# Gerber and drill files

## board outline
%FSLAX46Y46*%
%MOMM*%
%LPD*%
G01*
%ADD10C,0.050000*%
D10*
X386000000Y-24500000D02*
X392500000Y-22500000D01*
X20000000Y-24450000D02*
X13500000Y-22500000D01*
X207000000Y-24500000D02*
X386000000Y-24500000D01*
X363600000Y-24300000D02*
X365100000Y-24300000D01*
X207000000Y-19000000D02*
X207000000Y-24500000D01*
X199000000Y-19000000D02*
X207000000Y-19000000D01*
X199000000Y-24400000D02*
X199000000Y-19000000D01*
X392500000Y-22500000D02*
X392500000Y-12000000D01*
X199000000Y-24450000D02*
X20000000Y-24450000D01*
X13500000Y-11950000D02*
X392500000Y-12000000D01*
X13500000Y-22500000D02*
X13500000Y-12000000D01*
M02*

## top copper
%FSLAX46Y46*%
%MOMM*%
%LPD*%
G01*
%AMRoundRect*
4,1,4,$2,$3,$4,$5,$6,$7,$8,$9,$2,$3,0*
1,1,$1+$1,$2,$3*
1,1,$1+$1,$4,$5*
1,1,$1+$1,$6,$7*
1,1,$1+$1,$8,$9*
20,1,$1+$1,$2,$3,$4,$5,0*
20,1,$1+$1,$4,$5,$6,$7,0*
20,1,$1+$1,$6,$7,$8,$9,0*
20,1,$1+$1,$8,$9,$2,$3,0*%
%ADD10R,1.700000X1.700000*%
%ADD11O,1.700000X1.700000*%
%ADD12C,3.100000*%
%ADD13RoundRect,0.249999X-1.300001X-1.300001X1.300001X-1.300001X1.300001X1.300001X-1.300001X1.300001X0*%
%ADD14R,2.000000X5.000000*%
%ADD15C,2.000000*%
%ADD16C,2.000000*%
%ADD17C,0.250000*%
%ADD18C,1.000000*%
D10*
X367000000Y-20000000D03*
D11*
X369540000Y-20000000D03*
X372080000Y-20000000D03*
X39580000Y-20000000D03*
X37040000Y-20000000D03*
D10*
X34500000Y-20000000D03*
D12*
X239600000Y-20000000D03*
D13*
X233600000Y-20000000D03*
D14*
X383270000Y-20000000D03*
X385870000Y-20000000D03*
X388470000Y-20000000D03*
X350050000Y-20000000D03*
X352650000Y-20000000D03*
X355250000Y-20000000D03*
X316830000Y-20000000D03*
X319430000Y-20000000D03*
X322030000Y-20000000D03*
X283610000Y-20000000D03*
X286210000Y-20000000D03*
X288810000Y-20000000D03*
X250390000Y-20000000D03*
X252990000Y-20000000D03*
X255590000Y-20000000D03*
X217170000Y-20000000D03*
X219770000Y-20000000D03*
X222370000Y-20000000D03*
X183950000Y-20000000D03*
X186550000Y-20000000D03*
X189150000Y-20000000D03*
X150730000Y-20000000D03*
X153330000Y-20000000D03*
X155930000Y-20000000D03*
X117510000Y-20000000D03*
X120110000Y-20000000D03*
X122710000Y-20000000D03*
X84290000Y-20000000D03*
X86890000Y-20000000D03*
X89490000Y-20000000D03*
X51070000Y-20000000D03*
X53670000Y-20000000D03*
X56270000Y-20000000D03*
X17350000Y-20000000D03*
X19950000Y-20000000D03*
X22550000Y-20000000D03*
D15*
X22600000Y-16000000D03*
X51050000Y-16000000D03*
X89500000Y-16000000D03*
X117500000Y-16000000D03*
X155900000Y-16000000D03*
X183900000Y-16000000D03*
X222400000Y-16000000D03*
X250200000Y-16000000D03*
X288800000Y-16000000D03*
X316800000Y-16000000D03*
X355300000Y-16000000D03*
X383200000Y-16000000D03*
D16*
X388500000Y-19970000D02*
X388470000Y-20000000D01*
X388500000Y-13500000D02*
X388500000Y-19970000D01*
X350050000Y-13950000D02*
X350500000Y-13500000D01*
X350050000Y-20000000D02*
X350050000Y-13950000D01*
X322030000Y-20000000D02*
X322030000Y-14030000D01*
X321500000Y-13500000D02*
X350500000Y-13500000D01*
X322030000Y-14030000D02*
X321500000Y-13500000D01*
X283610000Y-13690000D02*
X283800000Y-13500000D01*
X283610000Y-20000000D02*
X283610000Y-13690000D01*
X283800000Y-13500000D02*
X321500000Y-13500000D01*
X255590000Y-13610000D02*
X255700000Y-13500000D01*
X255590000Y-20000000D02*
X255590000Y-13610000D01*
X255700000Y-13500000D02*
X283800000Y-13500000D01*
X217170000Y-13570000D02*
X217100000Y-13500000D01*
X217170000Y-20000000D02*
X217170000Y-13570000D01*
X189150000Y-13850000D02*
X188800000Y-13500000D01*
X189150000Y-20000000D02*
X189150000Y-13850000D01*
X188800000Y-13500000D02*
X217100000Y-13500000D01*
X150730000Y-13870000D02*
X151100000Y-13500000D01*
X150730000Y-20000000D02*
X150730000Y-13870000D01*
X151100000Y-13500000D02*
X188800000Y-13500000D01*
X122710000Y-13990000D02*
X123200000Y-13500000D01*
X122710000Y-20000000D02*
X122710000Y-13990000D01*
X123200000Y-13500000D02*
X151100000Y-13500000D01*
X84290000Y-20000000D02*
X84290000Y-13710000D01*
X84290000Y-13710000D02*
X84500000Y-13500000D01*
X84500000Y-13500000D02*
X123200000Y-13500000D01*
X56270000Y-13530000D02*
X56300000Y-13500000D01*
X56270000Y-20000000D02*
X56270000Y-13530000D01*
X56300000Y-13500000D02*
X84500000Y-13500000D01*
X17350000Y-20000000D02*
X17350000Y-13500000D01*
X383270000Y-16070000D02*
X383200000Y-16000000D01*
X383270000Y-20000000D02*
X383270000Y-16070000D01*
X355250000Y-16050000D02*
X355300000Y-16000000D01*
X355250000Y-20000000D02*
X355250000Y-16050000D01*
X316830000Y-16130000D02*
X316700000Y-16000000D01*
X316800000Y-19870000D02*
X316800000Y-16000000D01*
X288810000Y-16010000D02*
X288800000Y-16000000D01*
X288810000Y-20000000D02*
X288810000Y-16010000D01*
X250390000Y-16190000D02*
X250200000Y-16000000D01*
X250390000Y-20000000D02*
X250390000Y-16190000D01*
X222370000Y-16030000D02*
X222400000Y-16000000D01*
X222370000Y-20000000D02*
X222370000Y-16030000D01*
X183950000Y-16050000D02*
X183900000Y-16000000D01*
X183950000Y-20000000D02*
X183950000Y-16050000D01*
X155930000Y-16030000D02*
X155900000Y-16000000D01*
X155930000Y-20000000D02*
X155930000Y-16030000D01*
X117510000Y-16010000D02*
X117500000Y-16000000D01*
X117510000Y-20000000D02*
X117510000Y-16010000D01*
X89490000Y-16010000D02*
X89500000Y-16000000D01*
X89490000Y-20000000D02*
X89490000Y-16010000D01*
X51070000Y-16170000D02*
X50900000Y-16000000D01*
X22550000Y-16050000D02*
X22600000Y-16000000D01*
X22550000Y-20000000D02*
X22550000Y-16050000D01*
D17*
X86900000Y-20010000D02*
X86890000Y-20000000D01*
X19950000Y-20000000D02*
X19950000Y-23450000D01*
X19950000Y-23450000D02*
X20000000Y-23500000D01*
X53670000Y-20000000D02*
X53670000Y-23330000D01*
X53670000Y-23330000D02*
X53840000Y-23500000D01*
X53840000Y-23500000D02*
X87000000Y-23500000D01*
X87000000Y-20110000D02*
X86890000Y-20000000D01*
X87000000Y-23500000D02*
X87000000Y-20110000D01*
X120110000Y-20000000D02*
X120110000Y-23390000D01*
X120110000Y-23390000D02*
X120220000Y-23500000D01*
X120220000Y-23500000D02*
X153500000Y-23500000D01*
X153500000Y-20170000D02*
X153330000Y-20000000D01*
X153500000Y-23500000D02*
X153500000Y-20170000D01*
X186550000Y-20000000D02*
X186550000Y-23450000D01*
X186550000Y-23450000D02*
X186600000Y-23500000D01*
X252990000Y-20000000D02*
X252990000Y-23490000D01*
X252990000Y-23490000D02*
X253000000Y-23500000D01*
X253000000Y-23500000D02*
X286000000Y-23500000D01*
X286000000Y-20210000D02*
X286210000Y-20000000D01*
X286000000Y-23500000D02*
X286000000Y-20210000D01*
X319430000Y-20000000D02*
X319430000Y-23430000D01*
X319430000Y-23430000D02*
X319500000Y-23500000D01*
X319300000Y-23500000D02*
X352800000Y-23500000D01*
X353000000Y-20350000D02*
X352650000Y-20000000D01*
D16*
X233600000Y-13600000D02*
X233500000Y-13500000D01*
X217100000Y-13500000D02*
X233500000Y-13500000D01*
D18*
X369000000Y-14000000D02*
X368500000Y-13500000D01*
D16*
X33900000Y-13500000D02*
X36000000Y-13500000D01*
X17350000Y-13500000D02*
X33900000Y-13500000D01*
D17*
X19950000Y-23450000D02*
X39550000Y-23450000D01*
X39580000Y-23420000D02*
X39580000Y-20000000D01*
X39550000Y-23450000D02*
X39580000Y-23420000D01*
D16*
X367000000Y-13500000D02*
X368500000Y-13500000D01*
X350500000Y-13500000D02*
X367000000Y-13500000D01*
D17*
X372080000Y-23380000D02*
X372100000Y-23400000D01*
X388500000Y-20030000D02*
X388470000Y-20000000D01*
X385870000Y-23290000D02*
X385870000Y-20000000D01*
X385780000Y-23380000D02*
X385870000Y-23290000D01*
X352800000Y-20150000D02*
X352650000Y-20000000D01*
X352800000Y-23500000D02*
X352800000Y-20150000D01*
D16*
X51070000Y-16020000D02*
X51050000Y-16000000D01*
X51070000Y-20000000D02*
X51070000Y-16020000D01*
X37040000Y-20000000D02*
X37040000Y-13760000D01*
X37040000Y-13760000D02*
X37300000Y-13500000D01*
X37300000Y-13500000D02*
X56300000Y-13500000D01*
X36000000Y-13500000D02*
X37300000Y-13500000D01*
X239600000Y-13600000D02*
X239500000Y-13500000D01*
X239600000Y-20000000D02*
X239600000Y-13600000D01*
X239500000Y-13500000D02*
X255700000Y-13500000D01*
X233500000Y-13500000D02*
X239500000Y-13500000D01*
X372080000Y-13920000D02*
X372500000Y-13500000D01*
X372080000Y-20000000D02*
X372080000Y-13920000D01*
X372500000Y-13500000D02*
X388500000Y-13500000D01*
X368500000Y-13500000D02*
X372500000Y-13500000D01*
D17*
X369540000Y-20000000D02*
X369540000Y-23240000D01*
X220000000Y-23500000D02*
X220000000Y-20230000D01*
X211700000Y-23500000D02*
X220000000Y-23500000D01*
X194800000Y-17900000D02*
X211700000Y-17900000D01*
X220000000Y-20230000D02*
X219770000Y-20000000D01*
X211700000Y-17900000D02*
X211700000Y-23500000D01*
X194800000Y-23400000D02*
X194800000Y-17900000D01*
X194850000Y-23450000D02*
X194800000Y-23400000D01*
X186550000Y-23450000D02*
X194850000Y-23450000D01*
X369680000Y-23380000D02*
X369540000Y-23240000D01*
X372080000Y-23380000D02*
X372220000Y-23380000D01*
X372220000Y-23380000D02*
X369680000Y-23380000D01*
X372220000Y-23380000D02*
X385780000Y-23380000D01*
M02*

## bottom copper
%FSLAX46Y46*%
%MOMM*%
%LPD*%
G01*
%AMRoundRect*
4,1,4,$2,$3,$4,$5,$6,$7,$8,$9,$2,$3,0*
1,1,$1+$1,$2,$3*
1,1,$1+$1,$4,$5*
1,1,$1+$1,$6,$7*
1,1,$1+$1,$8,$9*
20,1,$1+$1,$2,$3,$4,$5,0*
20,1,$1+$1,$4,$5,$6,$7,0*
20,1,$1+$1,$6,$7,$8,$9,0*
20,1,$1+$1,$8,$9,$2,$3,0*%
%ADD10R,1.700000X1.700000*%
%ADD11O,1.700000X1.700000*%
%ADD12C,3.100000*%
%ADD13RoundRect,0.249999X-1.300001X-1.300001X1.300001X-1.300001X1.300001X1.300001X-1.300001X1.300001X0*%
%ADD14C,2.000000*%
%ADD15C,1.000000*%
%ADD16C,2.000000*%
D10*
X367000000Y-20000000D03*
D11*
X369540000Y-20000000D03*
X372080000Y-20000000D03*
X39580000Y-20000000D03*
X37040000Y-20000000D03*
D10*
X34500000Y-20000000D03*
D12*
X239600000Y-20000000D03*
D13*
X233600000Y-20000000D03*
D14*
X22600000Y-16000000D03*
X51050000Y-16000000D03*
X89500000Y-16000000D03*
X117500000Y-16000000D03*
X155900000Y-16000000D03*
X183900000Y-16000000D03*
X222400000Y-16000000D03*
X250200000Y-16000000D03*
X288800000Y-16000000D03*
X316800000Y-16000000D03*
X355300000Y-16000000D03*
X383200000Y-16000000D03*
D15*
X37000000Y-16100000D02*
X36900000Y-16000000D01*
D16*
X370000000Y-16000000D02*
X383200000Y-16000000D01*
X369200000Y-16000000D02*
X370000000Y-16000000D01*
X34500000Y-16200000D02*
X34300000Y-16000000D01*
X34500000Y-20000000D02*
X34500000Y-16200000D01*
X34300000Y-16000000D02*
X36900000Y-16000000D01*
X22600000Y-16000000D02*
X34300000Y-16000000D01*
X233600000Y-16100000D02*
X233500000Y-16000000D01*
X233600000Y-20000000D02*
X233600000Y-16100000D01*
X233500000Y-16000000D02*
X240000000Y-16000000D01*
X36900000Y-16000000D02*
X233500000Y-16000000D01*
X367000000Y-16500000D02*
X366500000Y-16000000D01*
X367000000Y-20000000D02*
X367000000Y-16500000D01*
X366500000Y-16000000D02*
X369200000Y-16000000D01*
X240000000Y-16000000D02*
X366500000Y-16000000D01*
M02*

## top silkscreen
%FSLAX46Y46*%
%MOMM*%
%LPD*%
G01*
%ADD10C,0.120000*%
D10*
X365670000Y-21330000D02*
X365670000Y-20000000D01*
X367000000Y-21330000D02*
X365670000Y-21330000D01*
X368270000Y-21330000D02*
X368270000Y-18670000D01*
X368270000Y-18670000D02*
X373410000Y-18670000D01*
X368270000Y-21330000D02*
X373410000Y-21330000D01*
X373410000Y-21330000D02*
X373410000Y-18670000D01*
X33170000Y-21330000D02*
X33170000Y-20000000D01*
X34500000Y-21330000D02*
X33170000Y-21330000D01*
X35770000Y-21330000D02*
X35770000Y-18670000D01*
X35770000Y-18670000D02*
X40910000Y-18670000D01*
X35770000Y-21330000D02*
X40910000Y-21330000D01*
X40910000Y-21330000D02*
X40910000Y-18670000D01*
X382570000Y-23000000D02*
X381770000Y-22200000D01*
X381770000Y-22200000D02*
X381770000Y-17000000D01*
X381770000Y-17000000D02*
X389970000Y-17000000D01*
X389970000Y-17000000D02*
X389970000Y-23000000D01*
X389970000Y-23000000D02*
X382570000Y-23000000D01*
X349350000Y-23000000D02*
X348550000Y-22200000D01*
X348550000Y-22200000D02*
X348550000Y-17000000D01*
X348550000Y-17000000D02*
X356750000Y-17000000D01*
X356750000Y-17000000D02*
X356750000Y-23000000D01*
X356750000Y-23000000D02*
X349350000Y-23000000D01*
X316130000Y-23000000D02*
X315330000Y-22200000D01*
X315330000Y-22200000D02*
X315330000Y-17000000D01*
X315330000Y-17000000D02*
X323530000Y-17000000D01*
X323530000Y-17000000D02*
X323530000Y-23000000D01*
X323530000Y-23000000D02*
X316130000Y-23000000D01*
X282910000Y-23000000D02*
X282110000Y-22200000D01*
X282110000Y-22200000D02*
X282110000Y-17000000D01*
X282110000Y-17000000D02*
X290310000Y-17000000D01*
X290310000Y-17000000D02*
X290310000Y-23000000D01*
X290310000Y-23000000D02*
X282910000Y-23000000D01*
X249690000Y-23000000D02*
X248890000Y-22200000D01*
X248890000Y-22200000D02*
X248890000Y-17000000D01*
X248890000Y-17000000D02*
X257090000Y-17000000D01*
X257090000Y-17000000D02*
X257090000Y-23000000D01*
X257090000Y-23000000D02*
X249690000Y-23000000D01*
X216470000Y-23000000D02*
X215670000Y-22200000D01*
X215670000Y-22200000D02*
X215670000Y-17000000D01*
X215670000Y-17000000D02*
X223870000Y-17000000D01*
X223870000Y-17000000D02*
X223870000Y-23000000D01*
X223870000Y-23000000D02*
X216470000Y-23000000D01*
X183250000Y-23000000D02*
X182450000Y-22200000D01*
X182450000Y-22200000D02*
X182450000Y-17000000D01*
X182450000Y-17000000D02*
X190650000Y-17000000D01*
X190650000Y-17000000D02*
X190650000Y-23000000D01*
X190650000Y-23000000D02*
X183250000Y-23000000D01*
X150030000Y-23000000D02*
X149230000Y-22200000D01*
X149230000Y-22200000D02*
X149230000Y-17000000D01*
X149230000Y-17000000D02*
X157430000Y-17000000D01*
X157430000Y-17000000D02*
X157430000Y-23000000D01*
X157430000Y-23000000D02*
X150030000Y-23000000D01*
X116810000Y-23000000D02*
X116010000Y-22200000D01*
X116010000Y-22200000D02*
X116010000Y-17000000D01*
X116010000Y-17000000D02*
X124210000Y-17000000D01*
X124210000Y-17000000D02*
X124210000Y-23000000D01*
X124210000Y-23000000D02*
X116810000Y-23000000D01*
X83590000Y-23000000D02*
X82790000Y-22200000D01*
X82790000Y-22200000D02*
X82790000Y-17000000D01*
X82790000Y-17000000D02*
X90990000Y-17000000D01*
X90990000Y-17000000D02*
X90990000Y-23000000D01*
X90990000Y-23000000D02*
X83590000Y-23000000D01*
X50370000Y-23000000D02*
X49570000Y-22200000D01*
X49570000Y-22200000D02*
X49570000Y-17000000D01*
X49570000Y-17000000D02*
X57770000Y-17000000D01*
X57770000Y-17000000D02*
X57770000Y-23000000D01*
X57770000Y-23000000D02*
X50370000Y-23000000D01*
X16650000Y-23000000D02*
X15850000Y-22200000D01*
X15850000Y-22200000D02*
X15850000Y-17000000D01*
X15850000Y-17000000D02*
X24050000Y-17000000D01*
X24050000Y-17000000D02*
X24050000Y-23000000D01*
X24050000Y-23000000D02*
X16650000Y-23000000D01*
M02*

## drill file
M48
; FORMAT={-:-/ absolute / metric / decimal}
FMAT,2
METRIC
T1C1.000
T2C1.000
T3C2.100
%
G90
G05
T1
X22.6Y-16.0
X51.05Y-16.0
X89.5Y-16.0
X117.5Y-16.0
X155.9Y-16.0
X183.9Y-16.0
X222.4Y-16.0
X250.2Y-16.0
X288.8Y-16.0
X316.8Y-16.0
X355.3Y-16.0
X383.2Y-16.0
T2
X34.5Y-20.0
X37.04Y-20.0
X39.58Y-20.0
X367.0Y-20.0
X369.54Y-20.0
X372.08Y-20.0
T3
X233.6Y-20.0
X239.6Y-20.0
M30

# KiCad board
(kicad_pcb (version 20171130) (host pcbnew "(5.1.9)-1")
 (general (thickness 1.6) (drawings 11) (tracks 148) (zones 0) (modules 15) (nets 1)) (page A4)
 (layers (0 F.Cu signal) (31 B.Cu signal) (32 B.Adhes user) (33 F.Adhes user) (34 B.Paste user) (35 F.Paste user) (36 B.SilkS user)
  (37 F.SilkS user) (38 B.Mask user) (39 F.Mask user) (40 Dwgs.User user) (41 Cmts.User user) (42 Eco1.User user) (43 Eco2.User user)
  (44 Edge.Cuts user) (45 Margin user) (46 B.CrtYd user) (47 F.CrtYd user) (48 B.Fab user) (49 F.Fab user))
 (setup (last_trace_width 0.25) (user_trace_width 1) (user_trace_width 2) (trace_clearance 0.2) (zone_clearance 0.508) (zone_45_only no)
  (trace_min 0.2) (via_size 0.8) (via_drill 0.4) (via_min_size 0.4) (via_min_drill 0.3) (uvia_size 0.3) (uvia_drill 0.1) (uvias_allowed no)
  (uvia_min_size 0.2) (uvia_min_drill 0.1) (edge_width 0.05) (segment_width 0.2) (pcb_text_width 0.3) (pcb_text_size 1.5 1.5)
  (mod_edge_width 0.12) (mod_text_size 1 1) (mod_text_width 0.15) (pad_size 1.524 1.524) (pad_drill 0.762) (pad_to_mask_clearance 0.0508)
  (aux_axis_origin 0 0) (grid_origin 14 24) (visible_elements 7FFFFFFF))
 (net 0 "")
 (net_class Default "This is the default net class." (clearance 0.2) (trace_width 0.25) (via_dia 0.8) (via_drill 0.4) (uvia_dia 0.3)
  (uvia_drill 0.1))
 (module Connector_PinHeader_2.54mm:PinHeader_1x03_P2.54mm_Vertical (layer F.Cu) (at 367 20 90)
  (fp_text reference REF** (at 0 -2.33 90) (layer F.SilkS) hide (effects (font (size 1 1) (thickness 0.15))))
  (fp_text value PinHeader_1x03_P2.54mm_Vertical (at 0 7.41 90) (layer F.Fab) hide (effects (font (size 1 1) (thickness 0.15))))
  (fp_line (start -1.33 -1.33) (end 0 -1.33) (layer F.SilkS) (width 0.12))
  (fp_line (start -1.33 0) (end -1.33 -1.33) (layer F.SilkS) (width 0.12))
  (fp_line (start -1.33 1.27) (end 1.33 1.27) (layer F.SilkS) (width 0.12))
  (fp_line (start 1.33 1.27) (end 1.33 6.41) (layer F.SilkS) (width 0.12))
  (fp_line (start -1.33 1.27) (end -1.33 6.41) (layer F.SilkS) (width 0.12))
  (fp_line (start -1.33 6.41) (end 1.33 6.41) (layer F.SilkS) (width 0.12))
  (pad 1 thru_hole rect (at 0 0 90) (size 1.7 1.7) (drill 1) (layers *.Cu *.Mask))
  (pad 2 thru_hole oval (at 0 2.54 90) (size 1.7 1.7) (drill 1) (layers *.Cu *.Mask))
  (pad 3 thru_hole oval (at 0 5.08 90) (size 1.7 1.7) (drill 1) (layers *.Cu *.Mask)))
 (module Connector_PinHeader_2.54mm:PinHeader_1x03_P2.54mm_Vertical (layer F.Cu) (at 34.5 20 90)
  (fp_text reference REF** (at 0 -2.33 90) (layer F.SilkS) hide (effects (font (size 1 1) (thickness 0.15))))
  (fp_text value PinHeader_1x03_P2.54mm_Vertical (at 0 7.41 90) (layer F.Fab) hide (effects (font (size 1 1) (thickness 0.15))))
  (fp_line (start -1.33 -1.33) (end 0 -1.33) (layer F.SilkS) (width 0.12))
  (fp_line (start -1.33 0) (end -1.33 -1.33) (layer F.SilkS) (width 0.12))
  (fp_line (start -1.33 1.27) (end 1.33 1.27) (layer F.SilkS) (width 0.12))
  (fp_line (start 1.33 1.27) (end 1.33 6.41) (layer F.SilkS) (width 0.12))
  (fp_line (start -1.33 1.27) (end -1.33 6.41) (layer F.SilkS) (width 0.12))
  (fp_line (start -1.33 6.41) (end 1.33 6.41) (layer F.SilkS) (width 0.12))
  (pad 3 thru_hole oval (at 0 5.08 90) (size 1.7 1.7) (drill 1) (layers *.Cu *.Mask))
  (pad 2 thru_hole oval (at 0 2.54 90) (size 1.7 1.7) (drill 1) (layers *.Cu *.Mask))
  (pad 1 thru_hole rect (at 0 0 90) (size 1.7 1.7) (drill 1) (layers *.Cu *.Mask)))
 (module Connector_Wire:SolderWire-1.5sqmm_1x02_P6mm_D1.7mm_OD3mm (layer F.Cu) (at 233.6 20)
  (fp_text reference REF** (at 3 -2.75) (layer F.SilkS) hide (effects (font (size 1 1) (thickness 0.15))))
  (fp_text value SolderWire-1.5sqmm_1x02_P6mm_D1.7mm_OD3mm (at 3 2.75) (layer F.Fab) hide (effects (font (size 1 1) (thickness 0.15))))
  (pad 2 thru_hole circle (at 6 0) (size 3.1 3.1) (drill 2.1) (layers *.Cu *.Mask))
  (pad 1 thru_hole roundrect (at 0 0) (size 3.1 3.1) (drill 2.1) (layers *.Cu *.Mask) (roundrect_rratio 0.08064499999999999)))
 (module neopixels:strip (layer F.Cu) (at 385.87 20)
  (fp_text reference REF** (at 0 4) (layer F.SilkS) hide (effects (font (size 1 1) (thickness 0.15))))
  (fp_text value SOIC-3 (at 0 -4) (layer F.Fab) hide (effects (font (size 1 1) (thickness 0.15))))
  (fp_line (start -3.3 3) (end -4.1 2.2) (layer F.SilkS) (width 0.12))
  (fp_line (start -4.1 2.2) (end -4.1 -3) (layer F.SilkS) (width 0.12))
  (fp_line (start -4.1 -3) (end 4.1 -3) (layer F.SilkS) (width 0.12))
  (fp_line (start 4.1 -3) (end 4.1 3) (layer F.SilkS) (width 0.12))
  (fp_line (start 4.1 3) (end -3.3 3) (layer F.SilkS) (width 0.12))
  (pad 1 smd rect (at -2.6 0) (size 2 5) (layers F.Cu F.Paste F.Mask))
  (pad 2 smd rect (at 0 0) (size 2 5) (layers F.Cu F.Paste F.Mask))
  (pad 3 smd rect (at 2.6 0) (size 2 5) (layers F.Cu F.Paste F.Mask)))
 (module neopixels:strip (layer F.Cu) (at 352.65 20)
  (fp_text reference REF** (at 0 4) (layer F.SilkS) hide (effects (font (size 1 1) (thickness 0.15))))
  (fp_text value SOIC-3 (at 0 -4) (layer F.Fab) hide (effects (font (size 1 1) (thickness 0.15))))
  (fp_line (start -3.3 3) (end -4.1 2.2) (layer F.SilkS) (width 0.12))
  (fp_line (start -4.1 2.2) (end -4.1 -3) (layer F.SilkS) (width 0.12))
  (fp_line (start -4.1 -3) (end 4.1 -3) (layer F.SilkS) (width 0.12))
  (fp_line (start 4.1 -3) (end 4.1 3) (layer F.SilkS) (width 0.12))
  (fp_line (start 4.1 3) (end -3.3 3) (layer F.SilkS) (width 0.12))
  (pad 1 smd rect (at -2.6 0) (size 2 5) (layers F.Cu F.Paste F.Mask))
  (pad 2 smd rect (at 0 0) (size 2 5) (layers F.Cu F.Paste F.Mask))
  (pad 3 smd rect (at 2.6 0) (size 2 5) (layers F.Cu F.Paste F.Mask)))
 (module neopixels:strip (layer F.Cu) (at 319.43 20)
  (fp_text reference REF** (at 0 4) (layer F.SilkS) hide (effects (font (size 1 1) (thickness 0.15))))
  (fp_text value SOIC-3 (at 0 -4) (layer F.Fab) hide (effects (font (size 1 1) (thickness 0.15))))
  (fp_line (start -3.3 3) (end -4.1 2.2) (layer F.SilkS) (width 0.12))
  (fp_line (start -4.1 2.2) (end -4.1 -3) (layer F.SilkS) (width 0.12))
  (fp_line (start -4.1 -3) (end 4.1 -3) (layer F.SilkS) (width 0.12))
  (fp_line (start 4.1 -3) (end 4.1 3) (layer F.SilkS) (width 0.12))
  (fp_line (start 4.1 3) (end -3.3 3) (layer F.SilkS) (width 0.12))
  (pad 1 smd rect (at -2.6 0) (size 2 5) (layers F.Cu F.Paste F.Mask))
  (pad 2 smd rect (at 0 0) (size 2 5) (layers F.Cu F.Paste F.Mask))
  (pad 3 smd rect (at 2.6 0) (size 2 5) (layers F.Cu F.Paste F.Mask)))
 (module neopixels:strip (layer F.Cu) (at 286.21 20)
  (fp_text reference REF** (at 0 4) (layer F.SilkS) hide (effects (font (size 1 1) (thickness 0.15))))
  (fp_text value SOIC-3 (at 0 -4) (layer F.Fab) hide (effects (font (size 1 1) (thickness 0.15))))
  (fp_line (start -3.3 3) (end -4.1 2.2) (layer F.SilkS) (width 0.12))
  (fp_line (start -4.1 2.2) (end -4.1 -3) (layer F.SilkS) (width 0.12))
  (fp_line (start -4.1 -3) (end 4.1 -3) (layer F.SilkS) (width 0.12))
  (fp_line (start 4.1 -3) (end 4.1 3) (layer F.SilkS) (width 0.12))
  (fp_line (start 4.1 3) (end -3.3 3) (layer F.SilkS) (width 0.12))
  (pad 1 smd rect (at -2.6 0) (size 2 5) (layers F.Cu F.Paste F.Mask))
  (pad 2 smd rect (at 0 0) (size 2 5) (layers F.Cu F.Paste F.Mask))
  (pad 3 smd rect (at 2.6 0) (size 2 5) (layers F.Cu F.Paste F.Mask)))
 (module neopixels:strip (layer F.Cu) (at 252.99 20)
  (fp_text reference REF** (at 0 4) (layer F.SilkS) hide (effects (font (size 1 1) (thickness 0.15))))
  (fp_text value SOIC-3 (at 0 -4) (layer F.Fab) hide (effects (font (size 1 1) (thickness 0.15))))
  (fp_line (start -3.3 3) (end -4.1 2.2) (layer F.SilkS) (width 0.12))
  (fp_line (start -4.1 2.2) (end -4.1 -3) (layer F.SilkS) (width 0.12))
  (fp_line (start -4.1 -3) (end 4.1 -3) (layer F.SilkS) (width 0.12))
  (fp_line (start 4.1 -3) (end 4.1 3) (layer F.SilkS) (width 0.12))
  (fp_line (start 4.1 3) (end -3.3 3) (layer F.SilkS) (width 0.12))
  (pad 1 smd rect (at -2.6 0) (size 2 5) (layers F.Cu F.Paste F.Mask))
  (pad 2 smd rect (at 0 0) (size 2 5) (layers F.Cu F.Paste F.Mask))
  (pad 3 smd rect (at 2.6 0) (size 2 5) (layers F.Cu F.Paste F.Mask)))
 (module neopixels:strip (layer F.Cu) (at 219.77 20)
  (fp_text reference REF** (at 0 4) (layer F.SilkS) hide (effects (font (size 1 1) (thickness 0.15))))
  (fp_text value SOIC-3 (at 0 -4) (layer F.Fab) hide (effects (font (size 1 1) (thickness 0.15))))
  (fp_line (start -3.3 3) (end -4.1 2.2) (layer F.SilkS) (width 0.12))
  (fp_line (start -4.1 2.2) (end -4.1 -3) (layer F.SilkS) (width 0.12))
  (fp_line (start -4.1 -3) (end 4.1 -3) (layer F.SilkS) (width 0.12))
  (fp_line (start 4.1 -3) (end 4.1 3) (layer F.SilkS) (width 0.12))
  (fp_line (start 4.1 3) (end -3.3 3) (layer F.SilkS) (width 0.12))
  (pad 1 smd rect (at -2.6 0) (size 2 5) (layers F.Cu F.Paste F.Mask))
  (pad 2 smd rect (at 0 0) (size 2 5) (layers F.Cu F.Paste F.Mask))
  (pad 3 smd rect (at 2.6 0) (size 2 5) (layers F.Cu F.Paste F.Mask)))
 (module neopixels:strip (layer F.Cu) (at 186.55 20)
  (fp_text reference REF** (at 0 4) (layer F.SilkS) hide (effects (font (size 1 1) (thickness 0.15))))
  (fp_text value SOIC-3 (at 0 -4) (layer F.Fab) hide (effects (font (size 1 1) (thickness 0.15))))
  (fp_line (start -3.3 3) (end -4.1 2.2) (layer F.SilkS) (width 0.12))
  (fp_line (start -4.1 2.2) (end -4.1 -3) (layer F.SilkS) (width 0.12))
  (fp_line (start -4.1 -3) (end 4.1 -3) (layer F.SilkS) (width 0.12))
  (fp_line (start 4.1 -3) (end 4.1 3) (layer F.SilkS) (width 0.12))
  (fp_line (start 4.1 3) (end -3.3 3) (layer F.SilkS) (width 0.12))
  (pad 1 smd rect (at -2.6 0) (size 2 5) (layers F.Cu F.Paste F.Mask))
  (pad 2 smd rect (at 0 0) (size 2 5) (layers F.Cu F.Paste F.Mask))
  (pad 3 smd rect (at 2.6 0) (size 2 5) (layers F.Cu F.Paste F.Mask)))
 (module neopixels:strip (layer F.Cu) (at 153.33 20)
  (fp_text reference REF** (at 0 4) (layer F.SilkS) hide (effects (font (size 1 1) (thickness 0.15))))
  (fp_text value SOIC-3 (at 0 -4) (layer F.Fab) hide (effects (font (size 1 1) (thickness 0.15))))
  (fp_line (start -3.3 3) (end -4.1 2.2) (layer F.SilkS) (width 0.12))
  (fp_line (start -4.1 2.2) (end -4.1 -3) (layer F.SilkS) (width 0.12))
  (fp_line (start -4.1 -3) (end 4.1 -3) (layer F.SilkS) (width 0.12))
  (fp_line (start 4.1 -3) (end 4.1 3) (layer F.SilkS) (width 0.12))
  (fp_line (start 4.1 3) (end -3.3 3) (layer F.SilkS) (width 0.12))
  (pad 1 smd rect (at -2.6 0) (size 2 5) (layers F.Cu F.Paste F.Mask))
  (pad 2 smd rect (at 0 0) (size 2 5) (layers F.Cu F.Paste F.Mask))
  (pad 3 smd rect (at 2.6 0) (size 2 5) (layers F.Cu F.Paste F.Mask)))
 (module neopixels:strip (layer F.Cu) (at 120.11 20)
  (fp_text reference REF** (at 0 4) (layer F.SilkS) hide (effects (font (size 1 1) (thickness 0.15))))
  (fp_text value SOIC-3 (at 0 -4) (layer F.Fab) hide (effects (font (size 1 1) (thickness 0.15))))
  (fp_line (start -3.3 3) (end -4.1 2.2) (layer F.SilkS) (width 0.12))
  (fp_line (start -4.1 2.2) (end -4.1 -3) (layer F.SilkS) (width 0.12))
  (fp_line (start -4.1 -3) (end 4.1 -3) (layer F.SilkS) (width 0.12))
  (fp_line (start 4.1 -3) (end 4.1 3) (layer F.SilkS) (width 0.12))
  (fp_line (start 4.1 3) (end -3.3 3) (layer F.SilkS) (width 0.12))
  (pad 1 smd rect (at -2.6 0) (size 2 5) (layers F.Cu F.Paste F.Mask))
  (pad 2 smd rect (at 0 0) (size 2 5) (layers F.Cu F.Paste F.Mask))
  (pad 3 smd rect (at 2.6 0) (size 2 5) (layers F.Cu F.Paste F.Mask)))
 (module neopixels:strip (layer F.Cu) (at 86.89 20)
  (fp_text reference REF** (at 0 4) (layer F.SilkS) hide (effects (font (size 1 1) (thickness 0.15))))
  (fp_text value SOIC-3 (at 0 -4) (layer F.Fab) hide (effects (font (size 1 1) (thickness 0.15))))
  (fp_line (start -3.3 3) (end -4.1 2.2) (layer F.SilkS) (width 0.12))
  (fp_line (start -4.1 2.2) (end -4.1 -3) (layer F.SilkS) (width 0.12))
  (fp_line (start -4.1 -3) (end 4.1 -3) (layer F.SilkS) (width 0.12))
  (fp_line (start 4.1 -3) (end 4.1 3) (layer F.SilkS) (width 0.12))
  (fp_line (start 4.1 3) (end -3.3 3) (layer F.SilkS) (width 0.12))
  (pad 1 smd rect (at -2.6 0) (size 2 5) (layers F.Cu F.Paste F.Mask))
  (pad 2 smd rect (at 0 0) (size 2 5) (layers F.Cu F.Paste F.Mask))
  (pad 3 smd rect (at 2.6 0) (size 2 5) (layers F.Cu F.Paste F.Mask)))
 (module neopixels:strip (layer F.Cu) (at 53.67 20)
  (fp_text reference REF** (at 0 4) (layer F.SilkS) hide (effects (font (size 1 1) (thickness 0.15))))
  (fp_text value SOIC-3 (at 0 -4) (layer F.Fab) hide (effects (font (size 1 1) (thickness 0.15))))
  (fp_line (start -3.3 3) (end -4.1 2.2) (layer F.SilkS) (width 0.12))
  (fp_line (start -4.1 2.2) (end -4.1 -3) (layer F.SilkS) (width 0.12))
  (fp_line (start -4.1 -3) (end 4.1 -3) (layer F.SilkS) (width 0.12))
  (fp_line (start 4.1 -3) (end 4.1 3) (layer F.SilkS) (width 0.12))
  (fp_line (start 4.1 3) (end -3.3 3) (layer F.SilkS) (width 0.12))
  (pad 1 smd rect (at -2.6 0) (size 2 5) (layers F.Cu F.Paste F.Mask))
  (pad 2 smd rect (at 0 0) (size 2 5) (layers F.Cu F.Paste F.Mask))
  (pad 3 smd rect (at 2.6 0) (size 2 5) (layers F.Cu F.Paste F.Mask)))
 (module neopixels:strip (layer F.Cu) (at 19.95 20)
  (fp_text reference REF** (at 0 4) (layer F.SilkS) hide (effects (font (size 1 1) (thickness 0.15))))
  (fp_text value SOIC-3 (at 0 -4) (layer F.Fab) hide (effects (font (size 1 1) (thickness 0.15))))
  (fp_line (start -3.3 3) (end -4.1 2.2) (layer F.SilkS) (width 0.12))
  (fp_line (start -4.1 2.2) (end -4.1 -3) (layer F.SilkS) (width 0.12))
  (fp_line (start -4.1 -3) (end 4.1 -3) (layer F.SilkS) (width 0.12))
  (fp_line (start 4.1 -3) (end 4.1 3) (layer F.SilkS) (width 0.12))
  (fp_line (start 4.1 3) (end -3.3 3) (layer F.SilkS) (width 0.12))
  (pad 1 smd rect (at -2.6 0) (size 2 5) (layers F.Cu F.Paste F.Mask))
  (pad 2 smd rect (at 0 0) (size 2 5) (layers F.Cu F.Paste F.Mask))
  (pad 3 smd rect (at 2.6 0) (size 2 5) (layers F.Cu F.Paste F.Mask)))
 (gr_line (start 386 24.5) (end 392.5 22.5) (layer Edge.Cuts) (width 0.05))
 (gr_line (start 20 24.45) (end 13.5 22.5) (layer Edge.Cuts) (width 0.05))
 (gr_line (start 207 24.5) (end 386 24.5) (layer Edge.Cuts) (width 0.05))
 (gr_line (start 363.6 24.3) (end 365.1 24.3) (layer Edge.Cuts) (width 0.05))
 (gr_line (start 207 19) (end 207 24.5) (layer Edge.Cuts) (width 0.05))
 (gr_line (start 199 19) (end 207 19) (layer Edge.Cuts) (width 0.05))
 (gr_line (start 199 24.4) (end 199 19) (layer Edge.Cuts) (width 0.05))
 (gr_line (start 392.5 22.5) (end 392.5 12) (layer Edge.Cuts) (width 0.05))
 (gr_line (start 199 24.45) (end 20 24.45) (layer Edge.Cuts) (width 0.05))
 (gr_line (start 13.5 11.95) (end 392.5 12) (layer Edge.Cuts) (width 0.05))
 (gr_line (start 13.5 22.5) (end 13.5 12) (layer Edge.Cuts) (width 0.05))
 (segment (start 388.5 19.97) (end 388.47 20) (width 2) (layer F.Cu) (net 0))
 (segment (start 388.5 13.5) (end 388.5 19.97) (width 2) (layer F.Cu) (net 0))
 (segment (start 350.05 13.95) (end 350.5 13.5) (width 2) (layer F.Cu) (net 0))
 (segment (start 350.05 20) (end 350.05 13.95) (width 2) (layer F.Cu) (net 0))
 (segment (start 322.03 20) (end 322.03 14.03) (width 2) (layer F.Cu) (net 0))
 (segment (start 321.5 13.5) (end 350.5 13.5) (width 2) (layer F.Cu) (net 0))
 (segment (start 322.03 14.03) (end 321.5 13.5) (width 2) (layer F.Cu) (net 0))
 (segment (start 283.61 13.69) (end 283.8 13.5) (width 2) (layer F.Cu) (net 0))
 (segment (start 283.61 20) (end 283.61 13.69) (width 2) (layer F.Cu) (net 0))
 (segment (start 283.8 13.5) (end 321.5 13.5) (width 2) (layer F.Cu) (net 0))
 (segment (start 255.59 13.61) (end 255.7 13.5) (width 2) (layer F.Cu) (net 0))
 (segment (start 255.59 20) (end 255.59 13.61) (width 2) (layer F.Cu) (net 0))
 (segment (start 255.7 13.5) (end 283.8 13.5) (width 2) (layer F.Cu) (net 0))
 (segment (start 217.17 13.57) (end 217.1 13.5) (width 2) (layer F.Cu) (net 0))
 (segment (start 217.17 20) (end 217.17 13.57) (width 2) (layer F.Cu) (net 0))
 (segment (start 189.15 13.85) (end 188.8 13.5) (width 2) (layer F.Cu) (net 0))
 (segment (start 189.15 20) (end 189.15 13.85) (width 2) (layer F.Cu) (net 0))
 (segment (start 188.8 13.5) (end 217.1 13.5) (width 2) (layer F.Cu) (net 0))
 (segment (start 150.73 13.87) (end 151.1 13.5) (width 2) (layer F.Cu) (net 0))
 (segment (start 150.73 20) (end 150.73 13.87) (width 2) (layer F.Cu) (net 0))
 (segment (start 151.1 13.5) (end 188.8 13.5) (width 2) (layer F.Cu) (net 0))
 (segment (start 122.71 13.99) (end 123.2 13.5) (width 2) (layer F.Cu) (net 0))
 (segment (start 122.71 20) (end 122.71 13.99) (width 2) (layer F.Cu) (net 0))
 (segment (start 123.2 13.5) (end 151.1 13.5) (width 2) (layer F.Cu) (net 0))
 (segment (start 84.29 20) (end 84.29 13.71) (width 2) (layer F.Cu) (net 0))
 (segment (start 84.29 13.71) (end 84.5 13.5) (width 2) (layer F.Cu) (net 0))
 (segment (start 84.5 13.5) (end 123.2 13.5) (width 2) (layer F.Cu) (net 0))
 (segment (start 56.27 13.53) (end 56.3 13.5) (width 2) (layer F.Cu) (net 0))
 (segment (start 56.27 20) (end 56.27 13.53) (width 2) (layer F.Cu) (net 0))
 (segment (start 56.3 13.5) (end 84.5 13.5) (width 2) (layer F.Cu) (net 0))
 (segment (start 17.35 20) (end 17.35 13.5) (width 2) (layer F.Cu) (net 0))
 (via (at 22.6 16) (size 2) (drill 1) (layers F.Cu B.Cu) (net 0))
 (via (at 51.05 16) (size 2) (drill 1) (layers F.Cu B.Cu) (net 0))
 (via (at 89.5 16) (size 2) (drill 1) (layers F.Cu B.Cu) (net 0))
 (via (at 117.5 16) (size 2) (drill 1) (layers F.Cu B.Cu) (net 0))
 (via (at 155.9 16) (size 2) (drill 1) (layers F.Cu B.Cu) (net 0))
 (via (at 183.9 16) (size 2) (drill 1) (layers F.Cu B.Cu) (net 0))
 (via (at 222.4 16) (size 2) (drill 1) (layers F.Cu B.Cu) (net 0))
 (via (at 250.2 16) (size 2) (drill 1) (layers F.Cu B.Cu) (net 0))
 (via (at 288.8 16) (size 2) (drill 1) (layers F.Cu B.Cu) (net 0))
 (via (at 316.8 16) (size 2) (drill 1) (layers F.Cu B.Cu) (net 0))
 (via (at 355.3 16) (size 2) (drill 1) (layers F.Cu B.Cu) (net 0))
 (via (at 383.2 16) (size 2) (drill 1) (layers F.Cu B.Cu) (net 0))
 (segment (start 383.27 16.07) (end 383.2 16) (width 2) (layer F.Cu) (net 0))
 (segment (start 383.27 20) (end 383.27 16.07) (width 2) (layer F.Cu) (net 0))
 (segment (start 355.25 16.05) (end 355.3 16) (width 2) (layer F.Cu) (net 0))
 (segment (start 355.25 20) (end 355.25 16.05) (width 2) (layer F.Cu) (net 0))
 (segment (start 316.83 16.13) (end 316.7 16) (width 2) (layer F.Cu) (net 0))
 (segment (start 316.8 19.87) (end 316.8 16) (width 2) (layer F.Cu) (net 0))
 (segment (start 288.81 16.01) (end 288.8 16) (width 2) (layer F.Cu) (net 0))
 (segment (start 288.81 20) (end 288.81 16.01) (width 2) (layer F.Cu) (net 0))
 (segment (start 250.39 16.19) (end 250.2 16) (width 2) (layer F.Cu) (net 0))
 (segment (start 250.39 20) (end 250.39 16.19) (width 2) (layer F.Cu) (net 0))
 (segment (start 222.37 16.03) (end 222.4 16) (width 2) (layer F.Cu) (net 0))
 (segment (start 222.37 20) (end 222.37 16.03) (width 2) (layer F.Cu) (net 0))
 (segment (start 183.95 16.05) (end 183.9 16) (width 2) (layer F.Cu) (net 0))
 (segment (start 183.95 20) (end 183.95 16.05) (width 2) (layer F.Cu) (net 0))
 (segment (start 155.93 16.03) (end 155.9 16) (width 2) (layer F.Cu) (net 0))
 (segment (start 155.93 20) (end 155.93 16.03) (width 2) (layer F.Cu) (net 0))
 (segment (start 117.51 16.01) (end 117.5 16) (width 2) (layer F.Cu) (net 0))
 (segment (start 117.51 20) (end 117.51 16.01) (width 2) (layer F.Cu) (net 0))
 (segment (start 89.49 16.01) (end 89.5 16) (width 2) (layer F.Cu) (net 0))
 (segment (start 89.49 20) (end 89.49 16.01) (width 2) (layer F.Cu) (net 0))
 (segment (start 51.07 16.17) (end 50.9 16) (width 2) (layer F.Cu) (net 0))
 (segment (start 22.55 16.05) (end 22.6 16) (width 2) (layer F.Cu) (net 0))
 (segment (start 22.55 20) (end 22.55 16.05) (width 2) (layer F.Cu) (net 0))
 (segment (start 37 16.1) (end 36.9 16) (width 1) (layer B.Cu) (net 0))
 (segment (start 86.9 20.01) (end 86.89 20) (width 0.25) (layer F.Cu) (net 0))
 (segment (start 19.95 20) (end 19.95 23.45) (width 0.25) (layer F.Cu) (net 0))
 (segment (start 19.95 23.45) (end 20 23.5) (width 0.25) (layer F.Cu) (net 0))
 (segment (start 53.67 20) (end 53.67 23.33) (width 0.25) (layer F.Cu) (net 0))
 (segment (start 53.67 23.33) (end 53.84 23.5) (width 0.25) (layer F.Cu) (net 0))
 (segment (start 53.84 23.5) (end 87 23.5) (width 0.25) (layer F.Cu) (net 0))
 (segment (start 87 20.11) (end 86.89 20) (width 0.25) (layer F.Cu) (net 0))
 (segment (start 87 23.5) (end 87 20.11) (width 0.25) (layer F.Cu) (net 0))
 (segment (start 120.11 20) (end 120.11 23.39) (width 0.25) (layer F.Cu) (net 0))
 (segment (start 120.11 23.39) (end 120.22 23.5) (width 0.25) (layer F.Cu) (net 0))
 (segment (start 120.22 23.5) (end 153.5 23.5) (width 0.25) (layer F.Cu) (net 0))
 (segment (start 153.5 20.17) (end 153.33 20) (width 0.25) (layer F.Cu) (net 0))
 (segment (start 153.5 23.5) (end 153.5 20.17) (width 0.25) (layer F.Cu) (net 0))
 (segment (start 186.55 20) (end 186.55 23.45) (width 0.25) (layer F.Cu) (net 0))
 (segment (start 186.55 23.45) (end 186.6 23.5) (width 0.25) (layer F.Cu) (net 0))
 (segment (start 252.99 20) (end 252.99 23.49) (width 0.25) (layer F.Cu) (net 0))
 (segment (start 252.99 23.49) (end 253 23.5) (width 0.25) (layer F.Cu) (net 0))
 (segment (start 253 23.5) (end 286 23.5) (width 0.25) (layer F.Cu) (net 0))
 (segment (start 286 20.21) (end 286.21 20) (width 0.25) (layer F.Cu) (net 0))
 (segment (start 286 23.5) (end 286 20.21) (width 0.25) (layer F.Cu) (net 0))
 (segment (start 319.43 20) (end 319.43 23.43) (width 0.25) (layer F.Cu) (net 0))
 (segment (start 319.43 23.43) (end 319.5 23.5) (width 0.25) (layer F.Cu) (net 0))
 (segment (start 319.3 23.5) (end 352.8 23.5) (width 0.25) (layer F.Cu) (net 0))
 (segment (start 353 20.35) (end 352.65 20) (width 0.25) (layer F.Cu) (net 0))
 (segment (start 233.6 13.6) (end 233.5 13.5) (width 2) (layer F.Cu) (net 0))
 (segment (start 217.1 13.5) (end 233.5 13.5) (width 2) (layer F.Cu) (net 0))
 (segment (start 369 14) (end 368.5 13.5) (width 1) (layer F.Cu) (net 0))
 (segment (start 370 16) (end 383.2 16) (width 2) (layer B.Cu) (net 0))
 (segment (start 33.9 13.5) (end 36 13.5) (width 2) (layer F.Cu) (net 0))
 (segment (start 17.35 13.5) (end 33.9 13.5) (width 2) (layer F.Cu) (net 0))
 (segment (start 19.95 23.45) (end 39.55 23.45) (width 0.25) (layer F.Cu) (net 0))
 (segment (start 39.58 23.42) (end 39.58 20) (width 0.25) (layer F.Cu) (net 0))
 (segment (start 39.55 23.45) (end 39.58 23.42) (width 0.25) (layer F.Cu) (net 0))
 (segment (start 367 13.5) (end 368.5 13.5) (width 2) (layer F.Cu) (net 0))
 (segment (start 350.5 13.5) (end 367 13.5) (width 2) (layer F.Cu) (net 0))
 (segment (start 369.2 16) (end 370 16) (width 2) (layer B.Cu) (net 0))
 (segment (start 372.08 23.38) (end 372.1 23.4) (width 0.25) (layer F.Cu) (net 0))
 (segment (start 388.5 20.03) (end 388.47 20) (width 0.25) (layer F.Cu) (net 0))
 (segment (start 385.87 23.29) (end 385.87 20) (width 0.25) (layer F.Cu) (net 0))
 (segment (start 385.78 23.38) (end 385.87 23.29) (width 0.25) (layer F.Cu) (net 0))
 (segment (start 352.8 20.15) (end 352.65 20) (width 0.25) (layer F.Cu) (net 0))
 (segment (start 352.8 23.5) (end 352.8 20.15) (width 0.25) (layer F.Cu) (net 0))
 (segment (start 51.07 16.02) (end 51.05 16) (width 2) (layer F.Cu) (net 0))
 (segment (start 51.07 20) (end 51.07 16.02) (width 2) (layer F.Cu) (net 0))
 (segment (start 34.5 16.2) (end 34.3 16) (width 2) (layer B.Cu) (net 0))
 (segment (start 34.5 20) (end 34.5 16.2) (width 2) (layer B.Cu) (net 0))
 (segment (start 34.3 16) (end 36.9 16) (width 2) (layer B.Cu) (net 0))
 (segment (start 22.6 16) (end 34.3 16) (width 2) (layer B.Cu) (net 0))
 (segment (start 37.04 20) (end 37.04 13.76) (width 2) (layer F.Cu) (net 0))
 (segment (start 37.04 13.76) (end 37.3 13.5) (width 2) (layer F.Cu) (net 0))
 (segment (start 37.3 13.5) (end 56.3 13.5) (width 2) (layer F.Cu) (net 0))
 (segment (start 36 13.5) (end 37.3 13.5) (width 2) (layer F.Cu) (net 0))
 (segment (start 233.6 16.1) (end 233.5 16) (width 2) (layer B.Cu) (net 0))
 (segment (start 233.6 20) (end 233.6 16.1) (width 2) (layer B.Cu) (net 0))
 (segment (start 233.5 16) (end 240 16) (width 2) (layer B.Cu) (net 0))
 (segment (start 36.9 16) (end 233.5 16) (width 2) (layer B.Cu) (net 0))
 (segment (start 239.6 13.6) (end 239.5 13.5) (width 2) (layer F.Cu) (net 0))
 (segment (start 239.6 20) (end 239.6 13.6) (width 2) (layer F.Cu) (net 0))
 (segment (start 239.5 13.5) (end 255.7 13.5) (width 2) (layer F.Cu) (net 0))
 (segment (start 233.5 13.5) (end 239.5 13.5) (width 2) (layer F.Cu) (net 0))
 (segment (start 367 16.5) (end 366.5 16) (width 2) (layer B.Cu) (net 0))
 (segment (start 367 20) (end 367 16.5) (width 2) (layer B.Cu) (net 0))
 (segment (start 366.5 16) (end 369.2 16) (width 2) (layer B.Cu) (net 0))
 (segment (start 240 16) (end 366.5 16) (width 2) (layer B.Cu) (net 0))
 (segment (start 372.08 13.92) (end 372.5 13.5) (width 2) (layer F.Cu) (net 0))
 (segment (start 372.08 20) (end 372.08 13.92) (width 2) (layer F.Cu) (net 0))
 (segment (start 372.5 13.5) (end 388.5 13.5) (width 2) (layer F.Cu) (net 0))
 (segment (start 368.5 13.5) (end 372.5 13.5) (width 2) (layer F.Cu) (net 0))
 (segment (start 369.54 20) (end 369.54 23.24) (width 0.25) (layer F.Cu) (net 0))
 (segment (start 220 23.5) (end 220 20.23) (width 0.25) (layer F.Cu) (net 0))
 (segment (start 211.7 23.5) (end 220 23.5) (width 0.25) (layer F.Cu) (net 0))
 (segment (start 194.8 17.9) (end 211.7 17.9) (width 0.25) (layer F.Cu) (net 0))
 (segment (start 220 20.23) (end 219.77 20) (width 0.25) (layer F.Cu) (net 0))
 (segment (start 211.7 17.9) (end 211.7 23.5) (width 0.25) (layer F.Cu) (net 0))
 (segment (start 194.8 23.4) (end 194.8 17.9) (width 0.25) (layer F.Cu) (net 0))
 (segment (start 194.85 23.45) (end 194.8 23.4) (width 0.25) (layer F.Cu) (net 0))
 (segment (start 186.55 23.45) (end 194.85 23.45) (width 0.25) (layer F.Cu) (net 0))
 (segment (start 369.68 23.38) (end 369.54 23.24) (width 0.25) (layer F.Cu) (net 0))
 (segment (start 372.08 23.38) (end 372.22 23.38) (width 0.25) (layer F.Cu) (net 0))
 (segment (start 372.22 23.38) (end 369.68 23.38) (width 0.25) (layer F.Cu) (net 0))
 (segment (start 372.22 23.38) (end 385.78 23.38) (width 0.25) (layer F.Cu) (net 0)))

